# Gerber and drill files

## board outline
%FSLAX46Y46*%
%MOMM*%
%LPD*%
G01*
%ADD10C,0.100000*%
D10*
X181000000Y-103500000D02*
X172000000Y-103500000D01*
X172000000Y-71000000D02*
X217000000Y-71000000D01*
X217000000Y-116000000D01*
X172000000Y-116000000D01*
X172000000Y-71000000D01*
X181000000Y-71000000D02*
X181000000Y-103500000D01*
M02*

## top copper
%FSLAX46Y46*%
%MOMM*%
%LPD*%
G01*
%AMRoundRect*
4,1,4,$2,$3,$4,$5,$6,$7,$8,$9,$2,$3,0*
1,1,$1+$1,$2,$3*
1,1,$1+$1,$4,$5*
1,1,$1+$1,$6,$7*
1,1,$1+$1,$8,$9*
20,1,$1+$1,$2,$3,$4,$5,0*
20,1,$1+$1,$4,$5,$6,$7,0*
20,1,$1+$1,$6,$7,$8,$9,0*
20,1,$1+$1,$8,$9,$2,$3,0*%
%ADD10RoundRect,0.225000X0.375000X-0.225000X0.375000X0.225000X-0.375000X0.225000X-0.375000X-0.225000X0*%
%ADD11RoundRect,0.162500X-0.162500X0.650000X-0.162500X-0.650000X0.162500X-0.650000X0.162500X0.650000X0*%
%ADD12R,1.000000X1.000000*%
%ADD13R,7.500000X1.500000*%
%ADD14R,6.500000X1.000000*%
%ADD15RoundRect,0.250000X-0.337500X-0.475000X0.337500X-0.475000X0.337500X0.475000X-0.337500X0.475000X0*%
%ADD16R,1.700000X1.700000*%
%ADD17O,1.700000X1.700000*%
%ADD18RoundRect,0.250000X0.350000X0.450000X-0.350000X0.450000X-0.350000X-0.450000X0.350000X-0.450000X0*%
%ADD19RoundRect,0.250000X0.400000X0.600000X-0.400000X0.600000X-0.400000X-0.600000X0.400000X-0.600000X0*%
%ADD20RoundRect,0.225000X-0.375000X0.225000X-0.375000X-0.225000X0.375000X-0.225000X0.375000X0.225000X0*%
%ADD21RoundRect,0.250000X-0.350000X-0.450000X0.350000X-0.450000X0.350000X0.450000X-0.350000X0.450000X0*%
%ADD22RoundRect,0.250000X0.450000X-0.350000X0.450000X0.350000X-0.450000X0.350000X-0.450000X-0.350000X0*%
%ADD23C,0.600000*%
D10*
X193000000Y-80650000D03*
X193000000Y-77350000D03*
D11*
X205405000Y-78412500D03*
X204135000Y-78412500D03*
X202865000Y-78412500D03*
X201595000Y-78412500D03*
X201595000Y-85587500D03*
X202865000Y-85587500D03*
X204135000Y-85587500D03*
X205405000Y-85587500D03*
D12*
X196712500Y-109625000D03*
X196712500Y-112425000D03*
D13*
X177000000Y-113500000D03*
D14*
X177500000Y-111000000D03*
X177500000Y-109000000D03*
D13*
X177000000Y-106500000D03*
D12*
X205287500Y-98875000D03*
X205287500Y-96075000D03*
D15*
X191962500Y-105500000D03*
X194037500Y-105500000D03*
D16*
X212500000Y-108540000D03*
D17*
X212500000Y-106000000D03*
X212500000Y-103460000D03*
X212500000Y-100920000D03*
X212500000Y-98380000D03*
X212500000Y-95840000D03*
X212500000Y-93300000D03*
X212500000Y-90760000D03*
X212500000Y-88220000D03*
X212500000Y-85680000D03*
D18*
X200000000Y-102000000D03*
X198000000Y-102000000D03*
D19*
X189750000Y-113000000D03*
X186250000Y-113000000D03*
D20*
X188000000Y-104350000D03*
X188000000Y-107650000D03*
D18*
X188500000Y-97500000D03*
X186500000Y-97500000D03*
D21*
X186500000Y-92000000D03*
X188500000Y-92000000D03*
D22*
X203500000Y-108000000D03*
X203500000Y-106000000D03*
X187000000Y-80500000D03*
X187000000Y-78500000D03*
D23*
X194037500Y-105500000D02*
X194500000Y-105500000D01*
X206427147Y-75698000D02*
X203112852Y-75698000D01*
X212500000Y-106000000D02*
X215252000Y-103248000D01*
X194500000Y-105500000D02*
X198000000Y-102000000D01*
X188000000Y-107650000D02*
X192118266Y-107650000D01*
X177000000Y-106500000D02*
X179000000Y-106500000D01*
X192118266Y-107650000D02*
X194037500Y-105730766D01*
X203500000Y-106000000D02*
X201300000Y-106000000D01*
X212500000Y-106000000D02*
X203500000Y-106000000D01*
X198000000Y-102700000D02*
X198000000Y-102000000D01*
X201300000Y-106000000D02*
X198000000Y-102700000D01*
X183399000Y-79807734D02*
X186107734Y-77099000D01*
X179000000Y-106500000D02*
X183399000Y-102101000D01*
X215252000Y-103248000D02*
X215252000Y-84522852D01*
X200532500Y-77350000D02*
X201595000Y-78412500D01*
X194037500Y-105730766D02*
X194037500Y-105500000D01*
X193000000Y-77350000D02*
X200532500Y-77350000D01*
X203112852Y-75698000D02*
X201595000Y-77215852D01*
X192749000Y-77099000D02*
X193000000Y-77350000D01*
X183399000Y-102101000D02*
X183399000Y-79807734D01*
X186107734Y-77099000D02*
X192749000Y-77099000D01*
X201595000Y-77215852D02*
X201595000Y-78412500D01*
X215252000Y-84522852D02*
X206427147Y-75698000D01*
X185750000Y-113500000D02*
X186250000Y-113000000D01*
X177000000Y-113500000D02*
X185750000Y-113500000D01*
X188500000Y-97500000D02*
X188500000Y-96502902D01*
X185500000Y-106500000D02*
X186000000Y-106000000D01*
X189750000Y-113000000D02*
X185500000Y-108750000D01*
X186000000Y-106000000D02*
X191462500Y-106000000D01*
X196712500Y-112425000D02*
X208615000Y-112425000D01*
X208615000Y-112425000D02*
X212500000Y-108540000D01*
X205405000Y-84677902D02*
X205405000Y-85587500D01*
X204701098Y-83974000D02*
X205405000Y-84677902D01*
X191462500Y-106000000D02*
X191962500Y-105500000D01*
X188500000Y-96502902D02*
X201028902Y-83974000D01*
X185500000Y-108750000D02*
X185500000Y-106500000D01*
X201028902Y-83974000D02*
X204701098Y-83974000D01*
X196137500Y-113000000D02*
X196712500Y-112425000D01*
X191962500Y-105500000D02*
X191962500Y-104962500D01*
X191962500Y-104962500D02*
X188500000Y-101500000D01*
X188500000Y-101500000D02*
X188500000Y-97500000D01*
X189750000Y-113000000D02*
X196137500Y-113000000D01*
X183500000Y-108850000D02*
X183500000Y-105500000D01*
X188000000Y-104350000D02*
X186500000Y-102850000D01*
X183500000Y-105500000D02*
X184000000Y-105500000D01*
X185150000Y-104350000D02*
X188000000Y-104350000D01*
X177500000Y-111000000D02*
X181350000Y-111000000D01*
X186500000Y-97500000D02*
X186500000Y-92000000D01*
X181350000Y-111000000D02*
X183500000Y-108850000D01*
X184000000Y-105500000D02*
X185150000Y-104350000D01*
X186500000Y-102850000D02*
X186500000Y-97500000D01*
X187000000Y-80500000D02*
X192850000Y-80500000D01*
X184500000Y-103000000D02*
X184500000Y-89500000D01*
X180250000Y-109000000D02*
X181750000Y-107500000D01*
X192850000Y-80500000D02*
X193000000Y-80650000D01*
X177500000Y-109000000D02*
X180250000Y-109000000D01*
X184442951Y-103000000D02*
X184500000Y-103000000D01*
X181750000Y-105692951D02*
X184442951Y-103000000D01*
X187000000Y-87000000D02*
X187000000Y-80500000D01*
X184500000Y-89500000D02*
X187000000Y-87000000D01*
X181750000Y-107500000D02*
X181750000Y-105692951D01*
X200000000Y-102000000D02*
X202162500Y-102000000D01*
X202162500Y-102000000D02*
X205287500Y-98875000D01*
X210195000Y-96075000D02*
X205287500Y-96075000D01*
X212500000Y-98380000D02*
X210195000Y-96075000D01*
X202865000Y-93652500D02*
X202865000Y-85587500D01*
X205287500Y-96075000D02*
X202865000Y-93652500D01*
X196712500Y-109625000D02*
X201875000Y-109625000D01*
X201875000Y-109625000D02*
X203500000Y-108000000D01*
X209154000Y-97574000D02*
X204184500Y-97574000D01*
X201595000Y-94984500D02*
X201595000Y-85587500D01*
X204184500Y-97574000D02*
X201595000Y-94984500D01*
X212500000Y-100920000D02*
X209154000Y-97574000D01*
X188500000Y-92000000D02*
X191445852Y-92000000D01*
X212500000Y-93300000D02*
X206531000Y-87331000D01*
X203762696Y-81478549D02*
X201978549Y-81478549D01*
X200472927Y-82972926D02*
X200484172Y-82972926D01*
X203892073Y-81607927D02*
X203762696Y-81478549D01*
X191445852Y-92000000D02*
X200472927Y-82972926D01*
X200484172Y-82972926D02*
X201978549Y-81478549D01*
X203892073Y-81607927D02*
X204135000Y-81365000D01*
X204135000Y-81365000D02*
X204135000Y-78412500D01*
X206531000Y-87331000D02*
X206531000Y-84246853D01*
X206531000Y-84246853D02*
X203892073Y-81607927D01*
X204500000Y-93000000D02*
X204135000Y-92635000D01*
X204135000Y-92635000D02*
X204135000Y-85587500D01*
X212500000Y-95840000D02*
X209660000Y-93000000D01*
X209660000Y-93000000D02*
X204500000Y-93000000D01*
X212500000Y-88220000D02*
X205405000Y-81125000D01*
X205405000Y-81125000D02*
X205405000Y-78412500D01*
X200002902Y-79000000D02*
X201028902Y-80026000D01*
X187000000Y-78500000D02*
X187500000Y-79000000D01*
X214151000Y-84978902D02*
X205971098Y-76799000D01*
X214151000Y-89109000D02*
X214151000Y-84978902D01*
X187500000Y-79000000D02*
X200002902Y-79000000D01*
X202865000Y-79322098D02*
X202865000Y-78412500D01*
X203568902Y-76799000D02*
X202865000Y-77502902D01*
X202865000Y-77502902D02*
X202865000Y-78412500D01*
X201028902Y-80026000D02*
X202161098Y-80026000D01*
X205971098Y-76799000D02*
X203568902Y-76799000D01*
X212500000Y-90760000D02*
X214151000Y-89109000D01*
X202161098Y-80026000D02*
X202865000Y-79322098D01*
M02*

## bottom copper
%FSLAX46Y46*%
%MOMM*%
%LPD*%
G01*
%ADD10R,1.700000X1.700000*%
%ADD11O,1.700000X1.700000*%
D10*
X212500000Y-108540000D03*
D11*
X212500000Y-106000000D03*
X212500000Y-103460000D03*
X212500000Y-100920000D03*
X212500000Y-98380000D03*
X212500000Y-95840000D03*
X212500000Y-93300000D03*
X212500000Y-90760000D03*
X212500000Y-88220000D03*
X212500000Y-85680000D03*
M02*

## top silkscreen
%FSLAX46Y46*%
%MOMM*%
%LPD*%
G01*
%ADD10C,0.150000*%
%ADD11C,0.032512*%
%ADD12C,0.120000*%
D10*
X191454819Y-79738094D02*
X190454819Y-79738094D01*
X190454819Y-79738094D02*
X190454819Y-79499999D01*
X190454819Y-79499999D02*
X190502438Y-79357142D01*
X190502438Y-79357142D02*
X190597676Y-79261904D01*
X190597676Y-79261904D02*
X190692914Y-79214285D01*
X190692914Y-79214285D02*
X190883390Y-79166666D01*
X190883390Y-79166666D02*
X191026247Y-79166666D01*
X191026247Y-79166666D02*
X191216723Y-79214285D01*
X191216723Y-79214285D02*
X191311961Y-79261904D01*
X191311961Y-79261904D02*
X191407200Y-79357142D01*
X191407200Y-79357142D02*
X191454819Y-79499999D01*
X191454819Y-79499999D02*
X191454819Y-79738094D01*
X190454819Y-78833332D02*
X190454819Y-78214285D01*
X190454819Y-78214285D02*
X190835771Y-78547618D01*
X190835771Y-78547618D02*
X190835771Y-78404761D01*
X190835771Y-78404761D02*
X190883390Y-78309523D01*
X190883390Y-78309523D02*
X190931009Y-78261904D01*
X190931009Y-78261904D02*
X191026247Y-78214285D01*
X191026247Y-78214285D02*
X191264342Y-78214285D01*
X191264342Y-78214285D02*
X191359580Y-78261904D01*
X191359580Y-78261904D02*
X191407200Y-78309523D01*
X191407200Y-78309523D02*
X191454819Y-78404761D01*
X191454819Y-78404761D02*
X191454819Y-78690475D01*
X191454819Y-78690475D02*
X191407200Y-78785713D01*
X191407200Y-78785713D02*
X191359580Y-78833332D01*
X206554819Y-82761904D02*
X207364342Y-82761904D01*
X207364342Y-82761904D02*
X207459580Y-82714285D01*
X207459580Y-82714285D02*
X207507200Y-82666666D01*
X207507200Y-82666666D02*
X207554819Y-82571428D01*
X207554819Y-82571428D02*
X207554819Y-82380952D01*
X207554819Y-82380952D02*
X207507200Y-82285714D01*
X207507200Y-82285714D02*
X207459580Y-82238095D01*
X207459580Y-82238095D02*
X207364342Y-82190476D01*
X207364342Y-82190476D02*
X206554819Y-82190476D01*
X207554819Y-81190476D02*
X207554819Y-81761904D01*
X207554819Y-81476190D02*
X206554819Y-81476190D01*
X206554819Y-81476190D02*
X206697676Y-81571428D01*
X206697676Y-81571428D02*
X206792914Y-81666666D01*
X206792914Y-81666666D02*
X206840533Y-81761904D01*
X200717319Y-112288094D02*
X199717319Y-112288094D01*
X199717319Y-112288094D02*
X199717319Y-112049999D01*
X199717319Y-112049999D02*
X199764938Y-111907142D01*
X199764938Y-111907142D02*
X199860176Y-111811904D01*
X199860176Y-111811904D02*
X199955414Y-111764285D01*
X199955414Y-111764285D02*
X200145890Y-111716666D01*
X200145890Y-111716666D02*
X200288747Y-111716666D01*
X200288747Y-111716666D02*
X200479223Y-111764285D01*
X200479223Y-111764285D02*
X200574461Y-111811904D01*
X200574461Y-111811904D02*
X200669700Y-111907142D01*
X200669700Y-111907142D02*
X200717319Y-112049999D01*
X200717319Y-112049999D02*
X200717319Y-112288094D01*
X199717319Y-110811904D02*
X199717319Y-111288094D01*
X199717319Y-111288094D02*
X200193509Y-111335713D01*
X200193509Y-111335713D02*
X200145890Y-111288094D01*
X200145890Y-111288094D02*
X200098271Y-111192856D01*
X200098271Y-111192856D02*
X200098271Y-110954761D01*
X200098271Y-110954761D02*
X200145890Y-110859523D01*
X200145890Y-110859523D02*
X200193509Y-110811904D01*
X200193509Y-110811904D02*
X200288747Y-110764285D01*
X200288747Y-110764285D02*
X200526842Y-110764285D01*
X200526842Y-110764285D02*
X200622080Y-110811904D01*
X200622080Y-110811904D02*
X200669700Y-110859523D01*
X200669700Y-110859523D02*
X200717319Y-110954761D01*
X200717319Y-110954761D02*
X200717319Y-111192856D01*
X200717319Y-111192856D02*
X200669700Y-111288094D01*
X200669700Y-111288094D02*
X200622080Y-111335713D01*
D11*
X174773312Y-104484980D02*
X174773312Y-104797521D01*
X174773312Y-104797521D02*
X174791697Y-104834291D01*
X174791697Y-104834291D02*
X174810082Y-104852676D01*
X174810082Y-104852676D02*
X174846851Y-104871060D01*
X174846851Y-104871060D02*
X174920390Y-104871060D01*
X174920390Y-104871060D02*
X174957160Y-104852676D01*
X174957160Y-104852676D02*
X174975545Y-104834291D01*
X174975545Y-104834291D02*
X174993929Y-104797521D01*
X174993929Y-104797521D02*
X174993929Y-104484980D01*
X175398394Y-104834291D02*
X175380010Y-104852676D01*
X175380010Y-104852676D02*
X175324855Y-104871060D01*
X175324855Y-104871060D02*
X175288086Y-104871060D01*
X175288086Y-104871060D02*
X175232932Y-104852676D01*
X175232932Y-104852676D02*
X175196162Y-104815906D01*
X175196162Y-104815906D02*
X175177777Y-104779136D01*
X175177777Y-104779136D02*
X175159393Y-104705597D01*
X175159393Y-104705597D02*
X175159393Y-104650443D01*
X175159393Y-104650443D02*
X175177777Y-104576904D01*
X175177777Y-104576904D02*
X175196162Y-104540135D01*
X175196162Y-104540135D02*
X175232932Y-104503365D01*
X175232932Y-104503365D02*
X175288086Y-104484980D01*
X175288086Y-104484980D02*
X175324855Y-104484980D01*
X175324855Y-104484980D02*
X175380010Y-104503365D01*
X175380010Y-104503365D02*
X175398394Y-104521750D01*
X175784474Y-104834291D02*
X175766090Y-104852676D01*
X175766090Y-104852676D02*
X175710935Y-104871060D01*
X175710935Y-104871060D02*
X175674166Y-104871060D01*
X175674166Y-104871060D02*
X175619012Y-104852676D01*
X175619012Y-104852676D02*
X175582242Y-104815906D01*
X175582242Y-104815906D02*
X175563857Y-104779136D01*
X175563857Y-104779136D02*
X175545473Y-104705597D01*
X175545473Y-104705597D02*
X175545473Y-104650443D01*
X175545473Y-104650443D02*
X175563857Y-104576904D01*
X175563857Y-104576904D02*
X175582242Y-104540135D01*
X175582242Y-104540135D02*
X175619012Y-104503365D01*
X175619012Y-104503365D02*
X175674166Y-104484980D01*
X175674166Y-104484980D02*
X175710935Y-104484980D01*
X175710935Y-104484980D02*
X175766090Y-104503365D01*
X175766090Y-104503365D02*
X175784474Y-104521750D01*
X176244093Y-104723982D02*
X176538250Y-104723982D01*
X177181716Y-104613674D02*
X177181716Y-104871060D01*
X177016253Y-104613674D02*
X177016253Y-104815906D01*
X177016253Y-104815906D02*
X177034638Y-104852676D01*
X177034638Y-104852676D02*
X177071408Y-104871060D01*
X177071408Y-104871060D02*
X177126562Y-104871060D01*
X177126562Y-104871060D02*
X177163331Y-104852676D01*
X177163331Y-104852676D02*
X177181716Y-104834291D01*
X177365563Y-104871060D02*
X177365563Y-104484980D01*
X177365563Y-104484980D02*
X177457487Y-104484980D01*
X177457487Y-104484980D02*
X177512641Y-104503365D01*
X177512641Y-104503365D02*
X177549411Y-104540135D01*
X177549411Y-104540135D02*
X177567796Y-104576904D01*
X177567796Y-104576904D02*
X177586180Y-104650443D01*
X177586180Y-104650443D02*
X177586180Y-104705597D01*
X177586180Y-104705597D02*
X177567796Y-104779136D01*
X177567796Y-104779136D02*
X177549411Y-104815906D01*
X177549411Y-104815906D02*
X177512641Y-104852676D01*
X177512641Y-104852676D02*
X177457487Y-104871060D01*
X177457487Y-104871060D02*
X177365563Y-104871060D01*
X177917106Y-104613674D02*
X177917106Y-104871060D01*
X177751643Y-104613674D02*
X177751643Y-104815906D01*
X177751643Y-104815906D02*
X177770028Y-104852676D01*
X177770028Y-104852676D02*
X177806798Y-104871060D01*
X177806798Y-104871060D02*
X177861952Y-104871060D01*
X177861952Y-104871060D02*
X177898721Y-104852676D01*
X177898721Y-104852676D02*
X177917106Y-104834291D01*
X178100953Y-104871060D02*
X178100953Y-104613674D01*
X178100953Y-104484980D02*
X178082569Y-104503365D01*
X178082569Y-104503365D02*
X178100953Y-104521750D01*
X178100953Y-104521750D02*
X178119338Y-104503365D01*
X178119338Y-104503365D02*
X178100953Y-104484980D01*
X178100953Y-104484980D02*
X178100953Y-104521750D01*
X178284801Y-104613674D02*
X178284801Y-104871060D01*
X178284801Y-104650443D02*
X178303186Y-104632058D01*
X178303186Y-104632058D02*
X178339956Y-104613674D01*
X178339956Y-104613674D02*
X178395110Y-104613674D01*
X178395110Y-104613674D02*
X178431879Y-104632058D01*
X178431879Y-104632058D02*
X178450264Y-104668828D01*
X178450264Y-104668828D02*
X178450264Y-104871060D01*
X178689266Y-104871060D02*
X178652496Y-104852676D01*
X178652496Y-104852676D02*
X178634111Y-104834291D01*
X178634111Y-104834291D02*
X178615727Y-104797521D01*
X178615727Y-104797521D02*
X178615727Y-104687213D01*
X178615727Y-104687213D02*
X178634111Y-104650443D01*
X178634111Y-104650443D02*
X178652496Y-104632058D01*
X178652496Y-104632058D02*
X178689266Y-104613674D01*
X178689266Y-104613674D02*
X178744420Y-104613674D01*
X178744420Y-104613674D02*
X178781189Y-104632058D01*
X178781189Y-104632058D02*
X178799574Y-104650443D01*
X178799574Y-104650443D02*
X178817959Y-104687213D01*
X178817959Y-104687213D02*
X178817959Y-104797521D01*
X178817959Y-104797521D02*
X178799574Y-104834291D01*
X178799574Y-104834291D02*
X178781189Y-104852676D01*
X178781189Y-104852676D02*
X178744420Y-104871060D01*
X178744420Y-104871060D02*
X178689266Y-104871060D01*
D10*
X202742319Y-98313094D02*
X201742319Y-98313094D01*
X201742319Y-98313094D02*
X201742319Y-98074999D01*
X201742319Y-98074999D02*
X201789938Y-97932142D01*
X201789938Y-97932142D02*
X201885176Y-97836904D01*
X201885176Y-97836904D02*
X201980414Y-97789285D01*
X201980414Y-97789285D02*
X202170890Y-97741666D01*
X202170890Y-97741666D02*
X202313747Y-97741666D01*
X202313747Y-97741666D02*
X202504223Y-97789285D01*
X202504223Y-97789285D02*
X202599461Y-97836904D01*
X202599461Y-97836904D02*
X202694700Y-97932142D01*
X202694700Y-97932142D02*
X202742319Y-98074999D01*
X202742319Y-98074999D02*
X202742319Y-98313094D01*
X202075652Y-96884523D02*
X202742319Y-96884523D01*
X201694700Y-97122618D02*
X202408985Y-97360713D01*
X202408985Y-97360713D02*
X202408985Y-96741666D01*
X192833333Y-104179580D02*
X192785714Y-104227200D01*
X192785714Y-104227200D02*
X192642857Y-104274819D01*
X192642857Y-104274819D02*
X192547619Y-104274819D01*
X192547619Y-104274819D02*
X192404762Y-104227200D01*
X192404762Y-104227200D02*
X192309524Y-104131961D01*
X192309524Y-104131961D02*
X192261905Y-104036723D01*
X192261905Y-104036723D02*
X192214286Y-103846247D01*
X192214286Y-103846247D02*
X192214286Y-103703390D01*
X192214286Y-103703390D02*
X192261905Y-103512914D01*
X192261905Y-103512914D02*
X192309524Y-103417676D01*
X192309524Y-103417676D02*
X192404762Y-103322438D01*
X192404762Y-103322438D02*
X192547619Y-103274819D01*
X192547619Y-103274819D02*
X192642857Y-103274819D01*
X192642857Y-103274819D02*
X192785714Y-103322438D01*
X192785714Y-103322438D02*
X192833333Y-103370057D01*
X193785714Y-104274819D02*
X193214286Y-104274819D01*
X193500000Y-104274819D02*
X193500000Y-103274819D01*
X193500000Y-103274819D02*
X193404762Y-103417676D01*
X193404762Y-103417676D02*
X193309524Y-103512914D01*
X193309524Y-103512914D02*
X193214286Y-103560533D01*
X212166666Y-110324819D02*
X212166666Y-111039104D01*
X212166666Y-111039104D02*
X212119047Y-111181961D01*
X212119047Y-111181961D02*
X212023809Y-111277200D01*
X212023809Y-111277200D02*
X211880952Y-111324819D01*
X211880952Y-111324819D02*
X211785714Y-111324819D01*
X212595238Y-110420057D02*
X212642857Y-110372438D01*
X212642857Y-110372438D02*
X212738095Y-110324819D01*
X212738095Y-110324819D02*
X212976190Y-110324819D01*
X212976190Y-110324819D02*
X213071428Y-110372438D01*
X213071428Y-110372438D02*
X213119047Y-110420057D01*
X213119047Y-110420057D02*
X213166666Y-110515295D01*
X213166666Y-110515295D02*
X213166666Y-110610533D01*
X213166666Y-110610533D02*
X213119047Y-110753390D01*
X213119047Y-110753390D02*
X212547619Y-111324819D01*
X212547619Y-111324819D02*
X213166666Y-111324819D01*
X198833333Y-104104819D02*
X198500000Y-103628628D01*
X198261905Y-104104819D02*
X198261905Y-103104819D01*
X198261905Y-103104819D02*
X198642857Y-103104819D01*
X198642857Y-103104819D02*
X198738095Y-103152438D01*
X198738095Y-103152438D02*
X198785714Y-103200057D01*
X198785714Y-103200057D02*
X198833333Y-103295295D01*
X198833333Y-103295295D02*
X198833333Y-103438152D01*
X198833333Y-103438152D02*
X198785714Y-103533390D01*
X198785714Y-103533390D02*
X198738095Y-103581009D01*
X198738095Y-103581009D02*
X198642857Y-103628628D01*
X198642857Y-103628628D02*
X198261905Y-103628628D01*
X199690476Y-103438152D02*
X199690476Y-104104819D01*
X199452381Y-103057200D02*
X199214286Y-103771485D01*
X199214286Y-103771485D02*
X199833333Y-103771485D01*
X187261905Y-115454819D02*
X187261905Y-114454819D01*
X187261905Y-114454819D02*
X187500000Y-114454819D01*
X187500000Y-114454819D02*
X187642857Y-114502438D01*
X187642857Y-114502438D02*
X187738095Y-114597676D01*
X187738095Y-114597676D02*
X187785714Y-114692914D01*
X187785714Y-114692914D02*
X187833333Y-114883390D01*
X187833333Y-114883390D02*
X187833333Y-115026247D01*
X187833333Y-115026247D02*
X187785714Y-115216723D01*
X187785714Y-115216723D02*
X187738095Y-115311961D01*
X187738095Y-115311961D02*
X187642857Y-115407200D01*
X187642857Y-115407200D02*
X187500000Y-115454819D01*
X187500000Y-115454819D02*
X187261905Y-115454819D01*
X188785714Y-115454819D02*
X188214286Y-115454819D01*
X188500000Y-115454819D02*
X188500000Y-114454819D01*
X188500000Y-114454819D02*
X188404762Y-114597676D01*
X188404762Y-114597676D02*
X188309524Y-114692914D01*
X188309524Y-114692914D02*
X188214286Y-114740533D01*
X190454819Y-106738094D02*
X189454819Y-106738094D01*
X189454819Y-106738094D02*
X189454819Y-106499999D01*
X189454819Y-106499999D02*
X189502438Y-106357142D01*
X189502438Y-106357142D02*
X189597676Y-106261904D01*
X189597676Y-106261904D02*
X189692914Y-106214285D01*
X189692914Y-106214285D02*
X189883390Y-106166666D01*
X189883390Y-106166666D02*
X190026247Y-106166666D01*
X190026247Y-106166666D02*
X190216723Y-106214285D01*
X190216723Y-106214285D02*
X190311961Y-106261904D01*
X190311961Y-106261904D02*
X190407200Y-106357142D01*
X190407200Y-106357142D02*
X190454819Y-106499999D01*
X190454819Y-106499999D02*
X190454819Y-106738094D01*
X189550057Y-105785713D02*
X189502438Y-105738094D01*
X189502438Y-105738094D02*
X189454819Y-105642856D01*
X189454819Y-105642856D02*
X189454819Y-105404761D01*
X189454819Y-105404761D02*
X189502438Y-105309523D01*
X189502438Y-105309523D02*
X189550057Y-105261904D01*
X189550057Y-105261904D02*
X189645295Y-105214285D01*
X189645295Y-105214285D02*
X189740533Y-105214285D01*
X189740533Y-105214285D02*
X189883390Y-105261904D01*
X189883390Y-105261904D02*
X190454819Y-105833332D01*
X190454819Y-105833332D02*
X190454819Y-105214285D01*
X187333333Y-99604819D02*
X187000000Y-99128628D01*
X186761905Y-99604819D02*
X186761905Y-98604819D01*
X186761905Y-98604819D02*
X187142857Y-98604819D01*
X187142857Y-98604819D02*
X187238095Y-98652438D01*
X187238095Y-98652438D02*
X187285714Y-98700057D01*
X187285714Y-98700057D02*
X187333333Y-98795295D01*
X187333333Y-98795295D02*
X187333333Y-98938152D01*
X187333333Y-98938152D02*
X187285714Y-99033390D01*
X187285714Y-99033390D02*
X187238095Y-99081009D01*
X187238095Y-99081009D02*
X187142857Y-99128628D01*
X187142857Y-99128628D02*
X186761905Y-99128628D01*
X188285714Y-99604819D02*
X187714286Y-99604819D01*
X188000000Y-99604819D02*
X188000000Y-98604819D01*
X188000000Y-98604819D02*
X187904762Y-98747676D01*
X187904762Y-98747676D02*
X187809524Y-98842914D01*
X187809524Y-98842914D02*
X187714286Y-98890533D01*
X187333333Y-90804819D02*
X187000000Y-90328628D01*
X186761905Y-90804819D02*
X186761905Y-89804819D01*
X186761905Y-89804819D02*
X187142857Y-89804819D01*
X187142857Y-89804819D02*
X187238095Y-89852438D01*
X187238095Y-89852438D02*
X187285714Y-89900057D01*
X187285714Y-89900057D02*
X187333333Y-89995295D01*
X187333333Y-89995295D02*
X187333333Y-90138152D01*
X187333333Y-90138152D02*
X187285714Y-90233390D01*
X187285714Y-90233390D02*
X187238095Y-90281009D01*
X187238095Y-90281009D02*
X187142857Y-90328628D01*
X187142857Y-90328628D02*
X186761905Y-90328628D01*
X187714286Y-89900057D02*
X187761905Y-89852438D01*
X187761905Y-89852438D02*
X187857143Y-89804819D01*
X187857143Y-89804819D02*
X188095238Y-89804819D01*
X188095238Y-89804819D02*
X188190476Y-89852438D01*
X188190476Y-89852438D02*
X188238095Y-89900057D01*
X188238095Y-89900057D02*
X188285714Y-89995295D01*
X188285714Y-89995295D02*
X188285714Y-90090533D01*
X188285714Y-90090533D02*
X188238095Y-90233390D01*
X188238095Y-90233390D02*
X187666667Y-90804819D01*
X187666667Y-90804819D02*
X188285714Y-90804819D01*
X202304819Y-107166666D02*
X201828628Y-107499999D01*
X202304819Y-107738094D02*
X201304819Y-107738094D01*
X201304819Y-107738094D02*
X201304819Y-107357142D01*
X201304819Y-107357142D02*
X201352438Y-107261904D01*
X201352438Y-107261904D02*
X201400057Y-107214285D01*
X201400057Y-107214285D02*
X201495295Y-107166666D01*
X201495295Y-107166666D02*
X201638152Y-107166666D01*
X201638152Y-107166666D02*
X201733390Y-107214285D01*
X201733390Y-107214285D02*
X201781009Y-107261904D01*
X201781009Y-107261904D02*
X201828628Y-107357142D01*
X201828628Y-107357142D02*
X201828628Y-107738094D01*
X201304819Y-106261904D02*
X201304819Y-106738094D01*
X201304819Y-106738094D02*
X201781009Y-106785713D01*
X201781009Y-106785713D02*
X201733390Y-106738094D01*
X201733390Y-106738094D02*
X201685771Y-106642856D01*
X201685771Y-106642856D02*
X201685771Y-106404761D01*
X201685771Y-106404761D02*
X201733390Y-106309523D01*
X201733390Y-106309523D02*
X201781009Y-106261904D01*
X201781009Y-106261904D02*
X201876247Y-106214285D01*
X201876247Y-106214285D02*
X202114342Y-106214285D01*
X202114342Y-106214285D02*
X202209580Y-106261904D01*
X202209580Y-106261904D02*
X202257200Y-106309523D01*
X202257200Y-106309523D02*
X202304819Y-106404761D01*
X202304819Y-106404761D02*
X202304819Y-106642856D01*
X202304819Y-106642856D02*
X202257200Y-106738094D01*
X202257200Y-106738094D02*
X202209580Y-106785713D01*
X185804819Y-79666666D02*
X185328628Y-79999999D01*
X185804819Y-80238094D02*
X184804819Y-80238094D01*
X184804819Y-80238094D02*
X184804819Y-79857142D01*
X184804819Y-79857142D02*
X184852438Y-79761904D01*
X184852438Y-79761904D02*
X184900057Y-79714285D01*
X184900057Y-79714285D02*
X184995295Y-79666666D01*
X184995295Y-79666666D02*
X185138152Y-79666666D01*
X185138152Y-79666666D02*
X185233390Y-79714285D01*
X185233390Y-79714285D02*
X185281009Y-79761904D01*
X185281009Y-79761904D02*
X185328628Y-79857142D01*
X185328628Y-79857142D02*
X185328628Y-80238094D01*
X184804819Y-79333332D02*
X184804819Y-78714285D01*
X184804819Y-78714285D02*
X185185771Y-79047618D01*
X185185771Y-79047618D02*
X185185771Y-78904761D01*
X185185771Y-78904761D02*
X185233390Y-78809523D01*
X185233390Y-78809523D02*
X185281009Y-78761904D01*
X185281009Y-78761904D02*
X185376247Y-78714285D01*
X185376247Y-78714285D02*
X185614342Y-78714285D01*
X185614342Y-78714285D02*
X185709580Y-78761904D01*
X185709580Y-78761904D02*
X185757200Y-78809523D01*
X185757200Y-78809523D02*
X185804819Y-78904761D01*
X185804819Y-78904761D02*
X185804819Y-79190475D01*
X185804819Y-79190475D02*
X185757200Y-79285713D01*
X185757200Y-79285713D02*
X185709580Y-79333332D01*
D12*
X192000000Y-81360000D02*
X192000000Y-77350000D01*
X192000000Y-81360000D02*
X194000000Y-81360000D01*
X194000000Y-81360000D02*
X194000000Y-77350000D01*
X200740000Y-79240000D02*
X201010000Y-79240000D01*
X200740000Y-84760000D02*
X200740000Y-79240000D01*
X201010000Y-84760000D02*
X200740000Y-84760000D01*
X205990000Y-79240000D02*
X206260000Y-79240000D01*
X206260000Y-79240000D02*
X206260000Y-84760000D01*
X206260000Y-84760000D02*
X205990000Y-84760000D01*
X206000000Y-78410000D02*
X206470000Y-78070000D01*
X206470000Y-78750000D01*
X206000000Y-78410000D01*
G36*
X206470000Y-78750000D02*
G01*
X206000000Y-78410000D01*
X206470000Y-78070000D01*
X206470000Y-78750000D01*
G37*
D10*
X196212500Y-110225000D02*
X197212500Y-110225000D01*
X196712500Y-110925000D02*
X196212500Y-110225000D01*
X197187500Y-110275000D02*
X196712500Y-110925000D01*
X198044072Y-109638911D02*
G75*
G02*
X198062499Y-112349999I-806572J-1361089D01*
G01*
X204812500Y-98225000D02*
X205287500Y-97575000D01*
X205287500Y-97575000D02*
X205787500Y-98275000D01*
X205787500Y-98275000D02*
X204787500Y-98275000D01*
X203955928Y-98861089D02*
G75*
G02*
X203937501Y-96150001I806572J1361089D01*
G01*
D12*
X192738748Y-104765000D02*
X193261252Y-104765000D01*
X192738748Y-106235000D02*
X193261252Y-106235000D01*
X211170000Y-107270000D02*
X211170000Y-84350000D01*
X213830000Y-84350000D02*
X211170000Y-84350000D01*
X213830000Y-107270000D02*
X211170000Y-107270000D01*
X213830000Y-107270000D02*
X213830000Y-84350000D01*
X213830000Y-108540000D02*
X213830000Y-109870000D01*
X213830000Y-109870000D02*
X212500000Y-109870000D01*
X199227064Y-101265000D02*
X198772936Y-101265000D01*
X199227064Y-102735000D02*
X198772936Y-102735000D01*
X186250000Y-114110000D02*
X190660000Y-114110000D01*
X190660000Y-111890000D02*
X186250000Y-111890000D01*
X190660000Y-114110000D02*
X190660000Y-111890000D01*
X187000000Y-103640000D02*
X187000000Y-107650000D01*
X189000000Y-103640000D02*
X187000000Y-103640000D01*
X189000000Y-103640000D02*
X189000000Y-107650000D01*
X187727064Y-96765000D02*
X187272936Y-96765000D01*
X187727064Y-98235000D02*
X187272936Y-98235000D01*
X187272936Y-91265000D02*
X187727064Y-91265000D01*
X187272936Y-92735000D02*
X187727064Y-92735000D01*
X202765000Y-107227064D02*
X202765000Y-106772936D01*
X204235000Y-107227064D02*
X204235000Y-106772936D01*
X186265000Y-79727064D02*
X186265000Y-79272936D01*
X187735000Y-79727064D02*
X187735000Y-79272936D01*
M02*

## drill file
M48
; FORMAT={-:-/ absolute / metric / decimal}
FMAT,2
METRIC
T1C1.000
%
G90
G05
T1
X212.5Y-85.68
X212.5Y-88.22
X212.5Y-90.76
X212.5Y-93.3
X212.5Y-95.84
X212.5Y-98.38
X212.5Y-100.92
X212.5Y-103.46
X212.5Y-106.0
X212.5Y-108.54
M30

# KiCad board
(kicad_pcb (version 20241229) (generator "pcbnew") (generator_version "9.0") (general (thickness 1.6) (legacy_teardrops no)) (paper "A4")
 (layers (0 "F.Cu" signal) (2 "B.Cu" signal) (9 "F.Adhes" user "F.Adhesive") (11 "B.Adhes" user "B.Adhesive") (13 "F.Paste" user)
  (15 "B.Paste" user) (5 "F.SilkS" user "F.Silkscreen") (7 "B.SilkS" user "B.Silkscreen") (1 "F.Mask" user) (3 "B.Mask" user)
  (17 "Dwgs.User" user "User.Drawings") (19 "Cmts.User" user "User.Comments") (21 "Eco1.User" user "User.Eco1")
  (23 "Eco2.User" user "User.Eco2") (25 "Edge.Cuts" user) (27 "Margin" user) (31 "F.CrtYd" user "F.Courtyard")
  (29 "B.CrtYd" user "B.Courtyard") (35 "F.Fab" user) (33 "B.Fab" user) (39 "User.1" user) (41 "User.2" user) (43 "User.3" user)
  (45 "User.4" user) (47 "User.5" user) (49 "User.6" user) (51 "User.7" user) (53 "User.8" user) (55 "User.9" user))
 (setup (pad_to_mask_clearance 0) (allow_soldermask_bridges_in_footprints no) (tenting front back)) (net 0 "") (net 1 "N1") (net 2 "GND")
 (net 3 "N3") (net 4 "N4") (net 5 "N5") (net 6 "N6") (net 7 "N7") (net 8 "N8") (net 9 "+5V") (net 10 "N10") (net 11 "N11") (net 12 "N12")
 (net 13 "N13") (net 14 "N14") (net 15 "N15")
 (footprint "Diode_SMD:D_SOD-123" (layer "F.Cu") (at 193 79 90)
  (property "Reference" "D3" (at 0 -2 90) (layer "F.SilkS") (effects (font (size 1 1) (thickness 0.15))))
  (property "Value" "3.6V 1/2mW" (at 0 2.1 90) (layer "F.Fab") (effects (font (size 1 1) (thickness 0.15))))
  (fp_line (start -2.36 -1) (end 1.65 -1) (stroke (width 0.12) (type solid)) (layer "F.SilkS"))
  (fp_line (start -2.36 -1) (end -2.36 1) (stroke (width 0.12) (type solid)) (layer "F.SilkS"))
  (fp_line (start -2.36 1) (end 1.65 1) (stroke (width 0.12) (type solid)) (layer "F.SilkS"))
  (pad "1" smd roundrect (at -1.65 0 90) (size 0.9 1.2) (layers "F.Cu" "F.Mask" "F.Paste") (roundrect_rratio 0.25) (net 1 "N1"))
  (pad "2" smd roundrect (at 1.65 0 90) (size 0.9 1.2) (layers "F.Cu" "F.Mask" "F.Paste") (roundrect_rratio 0.25) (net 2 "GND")))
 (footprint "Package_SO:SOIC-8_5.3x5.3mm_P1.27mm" (layer "F.Cu") (at 203.5 82 -90)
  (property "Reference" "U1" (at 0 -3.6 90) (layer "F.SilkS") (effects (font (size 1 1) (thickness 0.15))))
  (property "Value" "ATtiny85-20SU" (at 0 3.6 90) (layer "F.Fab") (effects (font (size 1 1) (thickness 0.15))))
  (fp_line (start -2.76 2.76) (end -2.76 2.49) (stroke (width 0.12) (type solid)) (layer "F.SilkS"))
  (fp_line (start 2.76 2.76) (end -2.76 2.76) (stroke (width 0.12) (type solid)) (layer "F.SilkS"))
  (fp_line (start 2.76 2.49) (end 2.76 2.76) (stroke (width 0.12) (type solid)) (layer "F.SilkS"))
  (fp_line (start -2.76 -2.49) (end -2.76 -2.76) (stroke (width 0.12) (type solid)) (layer "F.SilkS"))
  (fp_line (start -2.76 -2.76) (end 2.76 -2.76) (stroke (width 0.12) (type solid)) (layer "F.SilkS"))
  (fp_line (start 2.76 -2.76) (end 2.76 -2.49) (stroke (width 0.12) (type solid)) (layer "F.SilkS"))
  (fp_poly (pts (xy -3.59 -2.5) (xy -3.93 -2.97) (xy -3.25 -2.97)) (stroke (width 0.12) (type solid)) (fill yes) (layer "F.SilkS"))
  (pad "1" smd roundrect (at -3.5875 -1.905 270) (size 1.625 0.65) (layers "F.Cu" "F.Mask" "F.Paste") (roundrect_rratio 0.25) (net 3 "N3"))
  (pad "2" smd roundrect (at -3.5875 -0.635 270) (size 1.625 0.65) (layers "F.Cu" "F.Mask" "F.Paste") (roundrect_rratio 0.25) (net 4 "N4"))
  (pad "3" smd roundrect (at -3.5875 0.635 270) (size 1.625 0.65) (layers "F.Cu" "F.Mask" "F.Paste") (roundrect_rratio 0.25) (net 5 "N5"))
  (pad "4" smd roundrect (at -3.5875 1.905 270) (size 1.625 0.65) (layers "F.Cu" "F.Mask" "F.Paste") (roundrect_rratio 0.25) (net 2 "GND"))
  (pad "5" smd roundrect (at 3.5875 1.905 270) (size 1.625 0.65) (layers "F.Cu" "F.Mask" "F.Paste") (roundrect_rratio 0.25) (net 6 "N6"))
  (pad "6" smd roundrect (at 3.5875 0.635 270) (size 1.625 0.65) (layers "F.Cu" "F.Mask" "F.Paste") (roundrect_rratio 0.25) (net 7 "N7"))
  (pad "7" smd roundrect (at 3.5875 -0.635 270) (size 1.625 0.65) (layers "F.Cu" "F.Mask" "F.Paste") (roundrect_rratio 0.25) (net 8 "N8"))
  (pad "8" smd roundrect (at 3.5875 -1.905 270) (size 1.625 0.65) (layers "F.Cu" "F.Mask" "F.Paste") (roundrect_rratio 0.25) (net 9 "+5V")))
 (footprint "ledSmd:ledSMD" (layer "F.Cu") (at 196.7125 111.425 -90)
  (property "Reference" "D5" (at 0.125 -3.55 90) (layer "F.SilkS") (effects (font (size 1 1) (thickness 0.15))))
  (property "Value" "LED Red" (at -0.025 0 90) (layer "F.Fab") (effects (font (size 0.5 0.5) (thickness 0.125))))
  (fp_line (start -1.2 0.5) (end -1.2 -0.5) (stroke (width 0.15) (type solid)) (layer "F.SilkS"))
  (fp_line (start -0.5 0) (end -1.2 0.5) (stroke (width 0.15) (type solid)) (layer "F.SilkS"))
  (fp_line (start -1.15 -0.475) (end -0.5 0) (stroke (width 0.15) (type solid)) (layer "F.SilkS"))
  (fp_arc (start -1.786089 -1.331572) (mid -0.435753 -2.107089) (end 0.924999 -1.349999) (stroke (width 0.15) (type solid))
   (layer "F.SilkS"))
  (pad "1" smd rect (at -1.8 0 270) (size 1 1) (layers "F.Cu" "F.Mask" "F.Paste") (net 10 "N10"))
  (pad "2" smd rect (at 1 0 270) (size 1 1) (layers "F.Cu" "F.Mask" "F.Paste") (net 9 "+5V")))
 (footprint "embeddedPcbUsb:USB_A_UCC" (layer "F.Cu") (at 177.2 110)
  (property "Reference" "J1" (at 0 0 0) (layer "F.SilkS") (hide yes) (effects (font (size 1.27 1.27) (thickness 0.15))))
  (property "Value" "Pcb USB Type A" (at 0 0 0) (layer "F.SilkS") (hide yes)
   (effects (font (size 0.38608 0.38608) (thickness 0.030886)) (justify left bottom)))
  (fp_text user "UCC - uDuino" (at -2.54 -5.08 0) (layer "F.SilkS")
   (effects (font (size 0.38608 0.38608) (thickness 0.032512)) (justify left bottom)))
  (pad "1" smd rect (at -0.2 3.5) (size 7.5 1.5) (layers "F.Cu" "F.Mask" "F.Paste") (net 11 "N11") (solder_mask_margin 0.1016))
  (pad "2" smd rect (at 0.3 1) (size 6.5 1) (layers "F.Cu" "F.Mask" "F.Paste") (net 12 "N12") (solder_mask_margin 0.1016))
  (pad "3" smd rect (at 0.3 -1) (size 6.5 1) (layers "F.Cu" "F.Mask" "F.Paste") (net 1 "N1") (solder_mask_margin 0.1016))
  (pad "4" smd rect (at -0.2 -3.5) (size 7.5 1.5) (layers "F.Cu" "F.Mask" "F.Paste") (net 2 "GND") (solder_mask_margin 0.1016)))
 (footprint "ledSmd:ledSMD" (layer "F.Cu") (at 205.2875 97.075 90)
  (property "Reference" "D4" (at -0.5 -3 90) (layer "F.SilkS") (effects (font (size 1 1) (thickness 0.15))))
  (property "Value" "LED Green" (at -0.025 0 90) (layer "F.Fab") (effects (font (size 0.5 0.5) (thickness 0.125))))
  (fp_line (start -1.15 -0.475) (end -0.5 0) (stroke (width 0.15) (type solid)) (layer "F.SilkS"))
  (fp_line (start -0.5 0) (end -1.2 0.5) (stroke (width 0.15) (type solid)) (layer "F.SilkS"))
  (fp_line (start -1.2 0.5) (end -1.2 -0.5) (stroke (width 0.15) (type solid)) (layer "F.SilkS"))
  (fp_arc (start -1.786089 -1.331572) (mid -0.435753 -2.107089) (end 0.924999 -1.349999) (stroke (width 0.15) (type solid))
   (layer "F.SilkS"))
  (pad "1" smd rect (at -1.8 0 90) (size 1 1) (layers "F.Cu" "F.Mask" "F.Paste") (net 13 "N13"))
  (pad "2" smd rect (at 1 0 90) (size 1 1) (layers "F.Cu" "F.Mask" "F.Paste") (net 7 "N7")))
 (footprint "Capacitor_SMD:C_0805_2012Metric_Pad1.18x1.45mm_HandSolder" (layer "F.Cu") (at 193 105.5)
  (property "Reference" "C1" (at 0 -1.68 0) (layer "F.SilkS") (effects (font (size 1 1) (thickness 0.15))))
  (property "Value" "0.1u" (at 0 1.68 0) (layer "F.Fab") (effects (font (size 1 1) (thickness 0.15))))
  (fp_line (start -0.261252 -0.735) (end 0.261252 -0.735) (stroke (width 0.12) (type solid)) (layer "F.SilkS"))
  (fp_line (start -0.261252 0.735) (end 0.261252 0.735) (stroke (width 0.12) (type solid)) (layer "F.SilkS"))
  (pad "1" smd roundrect (at -1.0375 0) (size 1.175 1.45) (layers "F.Cu" "F.Mask" "F.Paste") (roundrect_rratio 0.212766) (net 9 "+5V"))
  (pad "2" smd roundrect (at 1.0375 0) (size 1.175 1.45) (layers "F.Cu" "F.Mask" "F.Paste") (roundrect_rratio 0.212766) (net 2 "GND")))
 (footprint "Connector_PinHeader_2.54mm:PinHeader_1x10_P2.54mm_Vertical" (layer "F.Cu") (at 212.5 108.54 180)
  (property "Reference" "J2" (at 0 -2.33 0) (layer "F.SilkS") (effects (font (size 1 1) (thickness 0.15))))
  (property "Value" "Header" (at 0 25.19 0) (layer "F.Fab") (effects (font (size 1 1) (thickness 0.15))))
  (fp_line (start 1.33 1.27) (end 1.33 24.19) (stroke (width 0.12) (type solid)) (layer "F.SilkS"))
  (fp_line (start -1.33 24.19) (end 1.33 24.19) (stroke (width 0.12) (type solid)) (layer "F.SilkS"))
  (fp_line (start -1.33 1.27) (end 1.33 1.27) (stroke (width 0.12) (type solid)) (layer "F.SilkS"))
  (fp_line (start -1.33 1.27) (end -1.33 24.19) (stroke (width 0.12) (type solid)) (layer "F.SilkS"))
  (fp_line (start -1.33 0) (end -1.33 -1.33) (stroke (width 0.12) (type solid)) (layer "F.SilkS"))
  (fp_line (start -1.33 -1.33) (end 0 -1.33) (stroke (width 0.12) (type solid)) (layer "F.SilkS"))
  (pad "1" thru_hole rect (at 0 0 180) (size 1.7 1.7) (drill 1) (layers "*.Cu" "*.Mask") (remove_unused_layers no) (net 9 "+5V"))
  (pad "2" thru_hole oval (at 0 2.54 180) (size 1.7 1.7) (drill 1) (layers "*.Cu" "*.Mask") (remove_unused_layers no) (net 2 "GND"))
  (pad "3" thru_hole oval (at 0 5.08 180) (size 1.7 1.7) (drill 1) (layers "*.Cu" "*.Mask") (remove_unused_layers no) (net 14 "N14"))
  (pad "4" thru_hole oval (at 0 7.62 180) (size 1.7 1.7) (drill 1) (layers "*.Cu" "*.Mask") (remove_unused_layers no) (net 6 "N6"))
  (pad "5" thru_hole oval (at 0 10.16 180) (size 1.7 1.7) (drill 1) (layers "*.Cu" "*.Mask") (remove_unused_layers no) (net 7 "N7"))
  (pad "6" thru_hole oval (at 0 12.7 180) (size 1.7 1.7) (drill 1) (layers "*.Cu" "*.Mask") (remove_unused_layers no) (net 8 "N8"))
  (pad "7" thru_hole oval (at 0 15.24 180) (size 1.7 1.7) (drill 1) (layers "*.Cu" "*.Mask") (remove_unused_layers no) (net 4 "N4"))
  (pad "8" thru_hole oval (at 0 17.78 180) (size 1.7 1.7) (drill 1) (layers "*.Cu" "*.Mask") (remove_unused_layers no) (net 5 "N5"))
  (pad "9" thru_hole oval (at 0 20.32 180) (size 1.7 1.7) (drill 1) (layers "*.Cu" "*.Mask") (remove_unused_layers no) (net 3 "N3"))
  (pad "10" thru_hole oval (at 0 22.86 180) (size 1.7 1.7) (drill 1) (layers "*.Cu" "*.Mask") (remove_unused_layers no) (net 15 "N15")))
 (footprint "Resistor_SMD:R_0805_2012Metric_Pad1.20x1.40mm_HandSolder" (layer "F.Cu") (at 199 102 180)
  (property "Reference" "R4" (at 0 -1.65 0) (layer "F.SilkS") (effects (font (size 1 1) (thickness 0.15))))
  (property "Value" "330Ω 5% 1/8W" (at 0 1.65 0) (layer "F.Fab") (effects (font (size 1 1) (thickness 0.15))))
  (fp_line (start -0.227064 0.735) (end 0.227064 0.735) (stroke (width 0.12) (type solid)) (layer "F.SilkS"))
  (fp_line (start -0.227064 -0.735) (end 0.227064 -0.735) (stroke (width 0.12) (type solid)) (layer "F.SilkS"))
  (pad "1" smd roundrect (at -1 0 180) (size 1.2 1.4) (layers "F.Cu" "F.Mask" "F.Paste") (roundrect_rratio 0.208333) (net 13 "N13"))
  (pad "2" smd roundrect (at 1 0 180) (size 1.2 1.4) (layers "F.Cu" "F.Mask" "F.Paste") (roundrect_rratio 0.208333) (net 2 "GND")))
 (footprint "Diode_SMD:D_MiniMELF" (layer "F.Cu") (at 188 113 180)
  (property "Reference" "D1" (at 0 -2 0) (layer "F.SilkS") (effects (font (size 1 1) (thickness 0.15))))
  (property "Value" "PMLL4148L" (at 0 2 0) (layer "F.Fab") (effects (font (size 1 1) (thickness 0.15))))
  (fp_line (start 1.75 -1.11) (end -2.66 -1.11) (stroke (width 0.12) (type solid)) (layer "F.SilkS"))
  (fp_line (start -2.66 1.11) (end 1.75 1.11) (stroke (width 0.12) (type solid)) (layer "F.SilkS"))
  (fp_line (start -2.66 -1.11) (end -2.66 1.11) (stroke (width 0.12) (type solid)) (layer "F.SilkS"))
  (pad "1" smd roundrect (at -1.75 0 180) (size 1.3 1.7) (layers "F.Cu" "F.Mask" "F.Paste") (roundrect_rratio 0.1923076923) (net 9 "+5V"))
  (pad "2" smd roundrect (at 1.75 0 180) (size 1.3 1.7) (layers "F.Cu" "F.Mask" "F.Paste") (roundrect_rratio 0.1923076923) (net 11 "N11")))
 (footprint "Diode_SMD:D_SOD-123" (layer "F.Cu") (at 188 106 -90)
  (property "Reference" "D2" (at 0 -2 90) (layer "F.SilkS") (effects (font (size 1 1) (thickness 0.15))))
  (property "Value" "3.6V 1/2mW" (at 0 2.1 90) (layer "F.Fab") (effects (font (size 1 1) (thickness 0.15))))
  (fp_line (start -2.36 1) (end 1.65 1) (stroke (width 0.12) (type solid)) (layer "F.SilkS"))
  (fp_line (start -2.36 -1) (end -2.36 1) (stroke (width 0.12) (type solid)) (layer "F.SilkS"))
  (fp_line (start -2.36 -1) (end 1.65 -1) (stroke (width 0.12) (type solid)) (layer "F.SilkS"))
  (pad "1" smd roundrect (at -1.65 0 270) (size 0.9 1.2) (layers "F.Cu" "F.Mask" "F.Paste") (roundrect_rratio 0.25) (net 12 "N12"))
  (pad "2" smd roundrect (at 1.65 0 270) (size 0.9 1.2) (layers "F.Cu" "F.Mask" "F.Paste") (roundrect_rratio 0.25) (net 2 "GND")))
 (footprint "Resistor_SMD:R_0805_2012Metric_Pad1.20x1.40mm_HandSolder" (layer "F.Cu") (at 187.5 97.5 180)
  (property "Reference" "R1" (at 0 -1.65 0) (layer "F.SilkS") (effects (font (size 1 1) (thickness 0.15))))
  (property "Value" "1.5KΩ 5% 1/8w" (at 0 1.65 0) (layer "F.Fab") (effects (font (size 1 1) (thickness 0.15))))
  (fp_line (start -0.227064 0.735) (end 0.227064 0.735) (stroke (width 0.12) (type solid)) (layer "F.SilkS"))
  (fp_line (start -0.227064 -0.735) (end 0.227064 -0.735) (stroke (width 0.12) (type solid)) (layer "F.SilkS"))
  (pad "1" smd roundrect (at -1 0 180) (size 1.2 1.4) (layers "F.Cu" "F.Mask" "F.Paste") (roundrect_rratio 0.208333) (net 9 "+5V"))
  (pad "2" smd roundrect (at 1 0 180) (size 1.2 1.4) (layers "F.Cu" "F.Mask" "F.Paste") (roundrect_rratio 0.208333) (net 12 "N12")))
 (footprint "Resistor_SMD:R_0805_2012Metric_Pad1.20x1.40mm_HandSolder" (layer "F.Cu") (at 187.5 92)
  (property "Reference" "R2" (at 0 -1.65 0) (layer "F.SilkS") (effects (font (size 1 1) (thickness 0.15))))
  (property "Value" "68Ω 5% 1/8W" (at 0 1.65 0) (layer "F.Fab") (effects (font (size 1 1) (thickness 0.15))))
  (fp_line (start -0.227064 -0.735) (end 0.227064 -0.735) (stroke (width 0.12) (type solid)) (layer "F.SilkS"))
  (fp_line (start -0.227064 0.735) (end 0.227064 0.735) (stroke (width 0.12) (type solid)) (layer "F.SilkS"))
  (pad "1" smd roundrect (at -1 0) (size 1.2 1.4) (layers "F.Cu" "F.Mask" "F.Paste") (roundrect_rratio 0.208333) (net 12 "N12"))
  (pad "2" smd roundrect (at 1 0) (size 1.2 1.4) (layers "F.Cu" "F.Mask" "F.Paste") (roundrect_rratio 0.208333) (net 4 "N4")))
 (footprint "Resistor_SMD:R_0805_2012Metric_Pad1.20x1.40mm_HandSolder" (layer "F.Cu") (at 203.5 107 90)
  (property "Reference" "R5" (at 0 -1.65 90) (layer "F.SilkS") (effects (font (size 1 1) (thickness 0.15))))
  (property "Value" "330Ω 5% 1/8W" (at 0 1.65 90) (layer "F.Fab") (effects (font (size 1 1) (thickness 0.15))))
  (fp_line (start -0.227064 -0.735) (end 0.227064 -0.735) (stroke (width 0.12) (type solid)) (layer "F.SilkS"))
  (fp_line (start -0.227064 0.735) (end 0.227064 0.735) (stroke (width 0.12) (type solid)) (layer "F.SilkS"))
  (pad "1" smd roundrect (at -1 0 90) (size 1.2 1.4) (layers "F.Cu" "F.Mask" "F.Paste") (roundrect_rratio 0.208333) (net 10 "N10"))
  (pad "2" smd roundrect (at 1 0 90) (size 1.2 1.4) (layers "F.Cu" "F.Mask" "F.Paste") (roundrect_rratio 0.208333) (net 2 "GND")))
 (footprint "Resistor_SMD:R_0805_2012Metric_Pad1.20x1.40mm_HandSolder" (layer "F.Cu") (at 187 79.5 90)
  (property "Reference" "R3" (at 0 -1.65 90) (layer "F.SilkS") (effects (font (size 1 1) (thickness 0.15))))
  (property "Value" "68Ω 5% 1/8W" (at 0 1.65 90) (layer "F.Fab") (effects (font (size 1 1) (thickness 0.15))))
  (fp_line (start -0.227064 -0.735) (end 0.227064 -0.735) (stroke (width 0.12) (type solid)) (layer "F.SilkS"))
  (fp_line (start -0.227064 0.735) (end 0.227064 0.735) (stroke (width 0.12) (type solid)) (layer "F.SilkS"))
  (pad "1" smd roundrect (at -1 0 90) (size 1.2 1.4) (layers "F.Cu" "F.Mask" "F.Paste") (roundrect_rratio 0.208333) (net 1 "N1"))
  (pad "2" smd roundrect (at 1 0 90) (size 1.2 1.4) (layers "F.Cu" "F.Mask" "F.Paste") (roundrect_rratio 0.208333) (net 5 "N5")))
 (gr_line (start 181 103.5) (end 172 103.5) (stroke (width 0.1) (type default)) (layer "Edge.Cuts"))
 (gr_rect (start 172 71) (end 217 116) (stroke (width 0.1) (type default)) (fill no) (layer "Edge.Cuts"))
 (gr_line (start 181 71) (end 181 103.5) (stroke (width 0.1) (type default)) (layer "Edge.Cuts"))
 (segment (start 194.0375 105.5) (end 194.5 105.5) (width 0.6) (layer "F.Cu") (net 2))
 (segment (start 206.427147 75.698) (end 203.112852 75.698) (width 0.6) (layer "F.Cu") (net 2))
 (segment (start 212.5 106) (end 215.252 103.248) (width 0.6) (layer "F.Cu") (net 2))
 (segment (start 194.5 105.5) (end 198 102) (width 0.6) (layer "F.Cu") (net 2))
 (segment (start 188 107.65) (end 192.118266 107.65) (width 0.6) (layer "F.Cu") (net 2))
 (segment (start 177 106.5) (end 179 106.5) (width 0.6) (layer "F.Cu") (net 2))
 (segment (start 192.118266 107.65) (end 194.0375 105.730766) (width 0.6) (layer "F.Cu") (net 2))
 (segment (start 203.5 106) (end 201.3 106) (width 0.6) (layer "F.Cu") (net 2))
 (segment (start 212.5 106) (end 203.5 106) (width 0.6) (layer "F.Cu") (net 2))
 (segment (start 198 102.7) (end 198 102) (width 0.6) (layer "F.Cu") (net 2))
 (segment (start 201.3 106) (end 198 102.7) (width 0.6) (layer "F.Cu") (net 2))
 (segment (start 183.399 79.807734) (end 186.107734 77.099) (width 0.6) (layer "F.Cu") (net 2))
 (segment (start 179 106.5) (end 183.399 102.101) (width 0.6) (layer "F.Cu") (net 2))
 (segment (start 215.252 103.248) (end 215.252 84.522852) (width 0.6) (layer "F.Cu") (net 2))
 (segment (start 200.5325 77.35) (end 201.595 78.4125) (width 0.6) (layer "F.Cu") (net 2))
 (segment (start 194.0375 105.730766) (end 194.0375 105.5) (width 0.6) (layer "F.Cu") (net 2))
 (segment (start 193 77.35) (end 200.5325 77.35) (width 0.6) (layer "F.Cu") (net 2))
 (segment (start 203.112852 75.698) (end 201.595 77.215852) (width 0.6) (layer "F.Cu") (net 2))
 (segment (start 192.749 77.099) (end 193 77.35) (width 0.6) (layer "F.Cu") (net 2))
 (segment (start 183.399 102.101) (end 183.399 79.807734) (width 0.6) (layer "F.Cu") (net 2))
 (segment (start 186.107734 77.099) (end 192.749 77.099) (width 0.6) (layer "F.Cu") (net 2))
 (segment (start 201.595 77.215852) (end 201.595 78.4125) (width 0.6) (layer "F.Cu") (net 2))
 (segment (start 215.252 84.522852) (end 206.427147 75.698) (width 0.6) (layer "F.Cu") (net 2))
 (segment (start 185.75 113.5) (end 186.25 113) (width 0.6) (layer "F.Cu") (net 11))
 (segment (start 177 113.5) (end 185.75 113.5) (width 0.6) (layer "F.Cu") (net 11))
 (segment (start 188.5 97.5) (end 188.5 96.502902) (width 0.6) (layer "F.Cu") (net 9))
 (segment (start 185.5 106.5) (end 186 106) (width 0.6) (layer "F.Cu") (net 9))
 (segment (start 189.75 113) (end 185.5 108.75) (width 0.6) (layer "F.Cu") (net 9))
 (segment (start 186 106) (end 191.4625 106) (width 0.6) (layer "F.Cu") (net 9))
 (segment (start 196.7125 112.425) (end 208.615 112.425) (width 0.6) (layer "F.Cu") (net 9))
 (segment (start 208.615 112.425) (end 212.5 108.54) (width 0.6) (layer "F.Cu") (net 9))
 (segment (start 205.405 84.677902) (end 205.405 85.5875) (width 0.6) (layer "F.Cu") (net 9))
 (segment (start 204.701098 83.974) (end 205.405 84.677902) (width 0.6) (layer "F.Cu") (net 9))
 (segment (start 191.4625 106) (end 191.9625 105.5) (width 0.6) (layer "F.Cu") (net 9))
 (segment (start 188.5 96.502902) (end 201.028902 83.974) (width 0.6) (layer "F.Cu") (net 9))
 (segment (start 185.5 108.75) (end 185.5 106.5) (width 0.6) (layer "F.Cu") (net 9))
 (segment (start 201.028902 83.974) (end 204.701098 83.974) (width 0.6) (layer "F.Cu") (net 9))
 (segment (start 196.1375 113) (end 196.7125 112.425) (width 0.6) (layer "F.Cu") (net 9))
 (segment (start 191.9625 105.5) (end 191.9625 104.9625) (width 0.6) (layer "F.Cu") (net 9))
 (segment (start 191.9625 104.9625) (end 188.5 101.5) (width 0.6) (layer "F.Cu") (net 9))
 (segment (start 188.5 101.5) (end 188.5 97.5) (width 0.6) (layer "F.Cu") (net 9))
 (segment (start 189.75 113) (end 196.1375 113) (width 0.6) (layer "F.Cu") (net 9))
 (segment (start 183.5 108.85) (end 183.5 105.5) (width 0.6) (layer "F.Cu") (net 12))
 (segment (start 188 104.35) (end 186.5 102.85) (width 0.6) (layer "F.Cu") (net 12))
 (segment (start 183.5 105.5) (end 184 105.5) (width 0.6) (layer "F.Cu") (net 12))
 (segment (start 185.15 104.35) (end 188 104.35) (width 0.6) (layer "F.Cu") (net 12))
 (segment (start 177.5 111) (end 181.35 111) (width 0.6) (layer "F.Cu") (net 12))
 (segment (start 186.5 97.5) (end 186.5 92) (width 0.6) (layer "F.Cu") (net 12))
 (segment (start 181.35 111) (end 183.5 108.85) (width 0.6) (layer "F.Cu") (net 12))
 (segment (start 184 105.5) (end 185.15 104.35) (width 0.6) (layer "F.Cu") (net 12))
 (segment (start 186.5 102.85) (end 186.5 97.5) (width 0.6) (layer "F.Cu") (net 12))
 (segment (start 187 80.5) (end 192.85 80.5) (width 0.6) (layer "F.Cu") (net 1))
 (segment (start 184.5 103) (end 184.5 89.5) (width 0.6) (layer "F.Cu") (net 1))
 (segment (start 180.25 109) (end 181.75 107.5) (width 0.6) (layer "F.Cu") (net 1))
 (segment (start 192.85 80.5) (end 193 80.65) (width 0.6) (layer "F.Cu") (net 1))
 (segment (start 177.5 109) (end 180.25 109) (width 0.6) (layer "F.Cu") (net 1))
 (segment (start 184.442951 103) (end 184.5 103) (width 0.6) (layer "F.Cu") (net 1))
 (segment (start 181.75 105.692951) (end 184.442951 103) (width 0.6) (layer "F.Cu") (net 1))
 (segment (start 187 87) (end 187 80.5) (width 0.6) (layer "F.Cu") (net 1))
 (segment (start 184.5 89.5) (end 187 87) (width 0.6) (layer "F.Cu") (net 1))
 (segment (start 181.75 107.5) (end 181.75 105.692951) (width 0.6) (layer "F.Cu") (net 1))
 (segment (start 200 102) (end 202.1625 102) (width 0.6) (layer "F.Cu") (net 13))
 (segment (start 202.1625 102) (end 205.2875 98.875) (width 0.6) (layer "F.Cu") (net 13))
 (segment (start 210.195 96.075) (end 205.2875 96.075) (width 0.6) (layer "F.Cu") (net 7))
 (segment (start 212.5 98.38) (end 210.195 96.075) (width 0.6) (layer "F.Cu") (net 7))
 (segment (start 202.865 93.6525) (end 202.865 85.5875) (width 0.6) (layer "F.Cu") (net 7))
 (segment (start 205.2875 96.075) (end 202.865 93.6525) (width 0.6) (layer "F.Cu") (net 7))
 (segment (start 196.7125 109.625) (end 201.875 109.625) (width 0.6) (layer "F.Cu") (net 10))
 (segment (start 201.875 109.625) (end 203.5 108) (width 0.6) (layer "F.Cu") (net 10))
 (segment (start 209.154 97.574) (end 204.1845 97.574) (width 0.6) (layer "F.Cu") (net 6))
 (segment (start 201.595 94.9845) (end 201.595 85.5875) (width 0.6) (layer "F.Cu") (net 6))
 (segment (start 204.1845 97.574) (end 201.595 94.9845) (width 0.6) (layer "F.Cu") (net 6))
 (segment (start 212.5 100.92) (end 209.154 97.574) (width 0.6) (layer "F.Cu") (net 6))
 (segment (start 188.5 92) (end 191.445852 92) (width 0.6) (layer "F.Cu") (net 4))
 (segment (start 212.5 93.3) (end 206.531 87.331) (width 0.6) (layer "F.Cu") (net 4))
 (segment (start 203.762696 81.478549) (end 201.978549 81.478549) (width 0.6) (layer "F.Cu") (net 4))
 (segment (start 200.472927 82.972926) (end 200.484172 82.972926) (width 0.6) (layer "F.Cu") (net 4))
 (segment (start 203.892073 81.607927) (end 203.762696 81.478549) (width 0.6) (layer "F.Cu") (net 4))
 (segment (start 191.445852 92) (end 200.472927 82.972926) (width 0.6) (layer "F.Cu") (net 4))
 (segment (start 200.484172 82.972926) (end 201.978549 81.478549) (width 0.6) (layer "F.Cu") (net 4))
 (segment (start 203.892073 81.607927) (end 204.135 81.365) (width 0.6) (layer "F.Cu") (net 4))
 (segment (start 204.135 81.365) (end 204.135 78.4125) (width 0.6) (layer "F.Cu") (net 4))
 (segment (start 206.531 87.331) (end 206.531 84.246853) (width 0.6) (layer "F.Cu") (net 4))
 (segment (start 206.531 84.246853) (end 203.892073 81.607927) (width 0.6) (layer "F.Cu") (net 4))
 (segment (start 204.5 93) (end 204.135 92.635) (width 0.6) (layer "F.Cu") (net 8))
 (segment (start 204.135 92.635) (end 204.135 85.5875) (width 0.6) (layer "F.Cu") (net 8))
 (segment (start 212.5 95.84) (end 209.66 93) (width 0.6) (layer "F.Cu") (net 8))
 (segment (start 209.66 93) (end 204.5 93) (width 0.6) (layer "F.Cu") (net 8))
 (segment (start 212.5 88.22) (end 205.405 81.125) (width 0.6) (layer "F.Cu") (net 3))
 (segment (start 205.405 81.125) (end 205.405 78.4125) (width 0.6) (layer "F.Cu") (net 3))
 (segment (start 200.002902 79) (end 201.028902 80.026) (width 0.6) (layer "F.Cu") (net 5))
 (segment (start 187 78.5) (end 187.5 79) (width 0.6) (layer "F.Cu") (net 5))
 (segment (start 214.151 84.978902) (end 205.971098 76.799) (width 0.6) (layer "F.Cu") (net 5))
 (segment (start 214.151 89.109) (end 214.151 84.978902) (width 0.6) (layer "F.Cu") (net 5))
 (segment (start 187.5 79) (end 200.002902 79) (width 0.6) (layer "F.Cu") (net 5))
 (segment (start 202.865 79.322098) (end 202.865 78.4125) (width 0.6) (layer "F.Cu") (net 5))
 (segment (start 203.568902 76.799) (end 202.865 77.502902) (width 0.6) (layer "F.Cu") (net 5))
 (segment (start 202.865 77.502902) (end 202.865 78.4125) (width 0.6) (layer "F.Cu") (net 5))
 (segment (start 201.028902 80.026) (end 202.161098 80.026) (width 0.6) (layer "F.Cu") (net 5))
 (segment (start 205.971098 76.799) (end 203.568902 76.799) (width 0.6) (layer "F.Cu") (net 5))
 (segment (start 212.5 90.76) (end 214.151 89.109) (width 0.6) (layer "F.Cu") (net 5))
 (segment (start 202.161098 80.026) (end 202.865 79.322098) (width 0.6) (layer "F.Cu") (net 5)))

